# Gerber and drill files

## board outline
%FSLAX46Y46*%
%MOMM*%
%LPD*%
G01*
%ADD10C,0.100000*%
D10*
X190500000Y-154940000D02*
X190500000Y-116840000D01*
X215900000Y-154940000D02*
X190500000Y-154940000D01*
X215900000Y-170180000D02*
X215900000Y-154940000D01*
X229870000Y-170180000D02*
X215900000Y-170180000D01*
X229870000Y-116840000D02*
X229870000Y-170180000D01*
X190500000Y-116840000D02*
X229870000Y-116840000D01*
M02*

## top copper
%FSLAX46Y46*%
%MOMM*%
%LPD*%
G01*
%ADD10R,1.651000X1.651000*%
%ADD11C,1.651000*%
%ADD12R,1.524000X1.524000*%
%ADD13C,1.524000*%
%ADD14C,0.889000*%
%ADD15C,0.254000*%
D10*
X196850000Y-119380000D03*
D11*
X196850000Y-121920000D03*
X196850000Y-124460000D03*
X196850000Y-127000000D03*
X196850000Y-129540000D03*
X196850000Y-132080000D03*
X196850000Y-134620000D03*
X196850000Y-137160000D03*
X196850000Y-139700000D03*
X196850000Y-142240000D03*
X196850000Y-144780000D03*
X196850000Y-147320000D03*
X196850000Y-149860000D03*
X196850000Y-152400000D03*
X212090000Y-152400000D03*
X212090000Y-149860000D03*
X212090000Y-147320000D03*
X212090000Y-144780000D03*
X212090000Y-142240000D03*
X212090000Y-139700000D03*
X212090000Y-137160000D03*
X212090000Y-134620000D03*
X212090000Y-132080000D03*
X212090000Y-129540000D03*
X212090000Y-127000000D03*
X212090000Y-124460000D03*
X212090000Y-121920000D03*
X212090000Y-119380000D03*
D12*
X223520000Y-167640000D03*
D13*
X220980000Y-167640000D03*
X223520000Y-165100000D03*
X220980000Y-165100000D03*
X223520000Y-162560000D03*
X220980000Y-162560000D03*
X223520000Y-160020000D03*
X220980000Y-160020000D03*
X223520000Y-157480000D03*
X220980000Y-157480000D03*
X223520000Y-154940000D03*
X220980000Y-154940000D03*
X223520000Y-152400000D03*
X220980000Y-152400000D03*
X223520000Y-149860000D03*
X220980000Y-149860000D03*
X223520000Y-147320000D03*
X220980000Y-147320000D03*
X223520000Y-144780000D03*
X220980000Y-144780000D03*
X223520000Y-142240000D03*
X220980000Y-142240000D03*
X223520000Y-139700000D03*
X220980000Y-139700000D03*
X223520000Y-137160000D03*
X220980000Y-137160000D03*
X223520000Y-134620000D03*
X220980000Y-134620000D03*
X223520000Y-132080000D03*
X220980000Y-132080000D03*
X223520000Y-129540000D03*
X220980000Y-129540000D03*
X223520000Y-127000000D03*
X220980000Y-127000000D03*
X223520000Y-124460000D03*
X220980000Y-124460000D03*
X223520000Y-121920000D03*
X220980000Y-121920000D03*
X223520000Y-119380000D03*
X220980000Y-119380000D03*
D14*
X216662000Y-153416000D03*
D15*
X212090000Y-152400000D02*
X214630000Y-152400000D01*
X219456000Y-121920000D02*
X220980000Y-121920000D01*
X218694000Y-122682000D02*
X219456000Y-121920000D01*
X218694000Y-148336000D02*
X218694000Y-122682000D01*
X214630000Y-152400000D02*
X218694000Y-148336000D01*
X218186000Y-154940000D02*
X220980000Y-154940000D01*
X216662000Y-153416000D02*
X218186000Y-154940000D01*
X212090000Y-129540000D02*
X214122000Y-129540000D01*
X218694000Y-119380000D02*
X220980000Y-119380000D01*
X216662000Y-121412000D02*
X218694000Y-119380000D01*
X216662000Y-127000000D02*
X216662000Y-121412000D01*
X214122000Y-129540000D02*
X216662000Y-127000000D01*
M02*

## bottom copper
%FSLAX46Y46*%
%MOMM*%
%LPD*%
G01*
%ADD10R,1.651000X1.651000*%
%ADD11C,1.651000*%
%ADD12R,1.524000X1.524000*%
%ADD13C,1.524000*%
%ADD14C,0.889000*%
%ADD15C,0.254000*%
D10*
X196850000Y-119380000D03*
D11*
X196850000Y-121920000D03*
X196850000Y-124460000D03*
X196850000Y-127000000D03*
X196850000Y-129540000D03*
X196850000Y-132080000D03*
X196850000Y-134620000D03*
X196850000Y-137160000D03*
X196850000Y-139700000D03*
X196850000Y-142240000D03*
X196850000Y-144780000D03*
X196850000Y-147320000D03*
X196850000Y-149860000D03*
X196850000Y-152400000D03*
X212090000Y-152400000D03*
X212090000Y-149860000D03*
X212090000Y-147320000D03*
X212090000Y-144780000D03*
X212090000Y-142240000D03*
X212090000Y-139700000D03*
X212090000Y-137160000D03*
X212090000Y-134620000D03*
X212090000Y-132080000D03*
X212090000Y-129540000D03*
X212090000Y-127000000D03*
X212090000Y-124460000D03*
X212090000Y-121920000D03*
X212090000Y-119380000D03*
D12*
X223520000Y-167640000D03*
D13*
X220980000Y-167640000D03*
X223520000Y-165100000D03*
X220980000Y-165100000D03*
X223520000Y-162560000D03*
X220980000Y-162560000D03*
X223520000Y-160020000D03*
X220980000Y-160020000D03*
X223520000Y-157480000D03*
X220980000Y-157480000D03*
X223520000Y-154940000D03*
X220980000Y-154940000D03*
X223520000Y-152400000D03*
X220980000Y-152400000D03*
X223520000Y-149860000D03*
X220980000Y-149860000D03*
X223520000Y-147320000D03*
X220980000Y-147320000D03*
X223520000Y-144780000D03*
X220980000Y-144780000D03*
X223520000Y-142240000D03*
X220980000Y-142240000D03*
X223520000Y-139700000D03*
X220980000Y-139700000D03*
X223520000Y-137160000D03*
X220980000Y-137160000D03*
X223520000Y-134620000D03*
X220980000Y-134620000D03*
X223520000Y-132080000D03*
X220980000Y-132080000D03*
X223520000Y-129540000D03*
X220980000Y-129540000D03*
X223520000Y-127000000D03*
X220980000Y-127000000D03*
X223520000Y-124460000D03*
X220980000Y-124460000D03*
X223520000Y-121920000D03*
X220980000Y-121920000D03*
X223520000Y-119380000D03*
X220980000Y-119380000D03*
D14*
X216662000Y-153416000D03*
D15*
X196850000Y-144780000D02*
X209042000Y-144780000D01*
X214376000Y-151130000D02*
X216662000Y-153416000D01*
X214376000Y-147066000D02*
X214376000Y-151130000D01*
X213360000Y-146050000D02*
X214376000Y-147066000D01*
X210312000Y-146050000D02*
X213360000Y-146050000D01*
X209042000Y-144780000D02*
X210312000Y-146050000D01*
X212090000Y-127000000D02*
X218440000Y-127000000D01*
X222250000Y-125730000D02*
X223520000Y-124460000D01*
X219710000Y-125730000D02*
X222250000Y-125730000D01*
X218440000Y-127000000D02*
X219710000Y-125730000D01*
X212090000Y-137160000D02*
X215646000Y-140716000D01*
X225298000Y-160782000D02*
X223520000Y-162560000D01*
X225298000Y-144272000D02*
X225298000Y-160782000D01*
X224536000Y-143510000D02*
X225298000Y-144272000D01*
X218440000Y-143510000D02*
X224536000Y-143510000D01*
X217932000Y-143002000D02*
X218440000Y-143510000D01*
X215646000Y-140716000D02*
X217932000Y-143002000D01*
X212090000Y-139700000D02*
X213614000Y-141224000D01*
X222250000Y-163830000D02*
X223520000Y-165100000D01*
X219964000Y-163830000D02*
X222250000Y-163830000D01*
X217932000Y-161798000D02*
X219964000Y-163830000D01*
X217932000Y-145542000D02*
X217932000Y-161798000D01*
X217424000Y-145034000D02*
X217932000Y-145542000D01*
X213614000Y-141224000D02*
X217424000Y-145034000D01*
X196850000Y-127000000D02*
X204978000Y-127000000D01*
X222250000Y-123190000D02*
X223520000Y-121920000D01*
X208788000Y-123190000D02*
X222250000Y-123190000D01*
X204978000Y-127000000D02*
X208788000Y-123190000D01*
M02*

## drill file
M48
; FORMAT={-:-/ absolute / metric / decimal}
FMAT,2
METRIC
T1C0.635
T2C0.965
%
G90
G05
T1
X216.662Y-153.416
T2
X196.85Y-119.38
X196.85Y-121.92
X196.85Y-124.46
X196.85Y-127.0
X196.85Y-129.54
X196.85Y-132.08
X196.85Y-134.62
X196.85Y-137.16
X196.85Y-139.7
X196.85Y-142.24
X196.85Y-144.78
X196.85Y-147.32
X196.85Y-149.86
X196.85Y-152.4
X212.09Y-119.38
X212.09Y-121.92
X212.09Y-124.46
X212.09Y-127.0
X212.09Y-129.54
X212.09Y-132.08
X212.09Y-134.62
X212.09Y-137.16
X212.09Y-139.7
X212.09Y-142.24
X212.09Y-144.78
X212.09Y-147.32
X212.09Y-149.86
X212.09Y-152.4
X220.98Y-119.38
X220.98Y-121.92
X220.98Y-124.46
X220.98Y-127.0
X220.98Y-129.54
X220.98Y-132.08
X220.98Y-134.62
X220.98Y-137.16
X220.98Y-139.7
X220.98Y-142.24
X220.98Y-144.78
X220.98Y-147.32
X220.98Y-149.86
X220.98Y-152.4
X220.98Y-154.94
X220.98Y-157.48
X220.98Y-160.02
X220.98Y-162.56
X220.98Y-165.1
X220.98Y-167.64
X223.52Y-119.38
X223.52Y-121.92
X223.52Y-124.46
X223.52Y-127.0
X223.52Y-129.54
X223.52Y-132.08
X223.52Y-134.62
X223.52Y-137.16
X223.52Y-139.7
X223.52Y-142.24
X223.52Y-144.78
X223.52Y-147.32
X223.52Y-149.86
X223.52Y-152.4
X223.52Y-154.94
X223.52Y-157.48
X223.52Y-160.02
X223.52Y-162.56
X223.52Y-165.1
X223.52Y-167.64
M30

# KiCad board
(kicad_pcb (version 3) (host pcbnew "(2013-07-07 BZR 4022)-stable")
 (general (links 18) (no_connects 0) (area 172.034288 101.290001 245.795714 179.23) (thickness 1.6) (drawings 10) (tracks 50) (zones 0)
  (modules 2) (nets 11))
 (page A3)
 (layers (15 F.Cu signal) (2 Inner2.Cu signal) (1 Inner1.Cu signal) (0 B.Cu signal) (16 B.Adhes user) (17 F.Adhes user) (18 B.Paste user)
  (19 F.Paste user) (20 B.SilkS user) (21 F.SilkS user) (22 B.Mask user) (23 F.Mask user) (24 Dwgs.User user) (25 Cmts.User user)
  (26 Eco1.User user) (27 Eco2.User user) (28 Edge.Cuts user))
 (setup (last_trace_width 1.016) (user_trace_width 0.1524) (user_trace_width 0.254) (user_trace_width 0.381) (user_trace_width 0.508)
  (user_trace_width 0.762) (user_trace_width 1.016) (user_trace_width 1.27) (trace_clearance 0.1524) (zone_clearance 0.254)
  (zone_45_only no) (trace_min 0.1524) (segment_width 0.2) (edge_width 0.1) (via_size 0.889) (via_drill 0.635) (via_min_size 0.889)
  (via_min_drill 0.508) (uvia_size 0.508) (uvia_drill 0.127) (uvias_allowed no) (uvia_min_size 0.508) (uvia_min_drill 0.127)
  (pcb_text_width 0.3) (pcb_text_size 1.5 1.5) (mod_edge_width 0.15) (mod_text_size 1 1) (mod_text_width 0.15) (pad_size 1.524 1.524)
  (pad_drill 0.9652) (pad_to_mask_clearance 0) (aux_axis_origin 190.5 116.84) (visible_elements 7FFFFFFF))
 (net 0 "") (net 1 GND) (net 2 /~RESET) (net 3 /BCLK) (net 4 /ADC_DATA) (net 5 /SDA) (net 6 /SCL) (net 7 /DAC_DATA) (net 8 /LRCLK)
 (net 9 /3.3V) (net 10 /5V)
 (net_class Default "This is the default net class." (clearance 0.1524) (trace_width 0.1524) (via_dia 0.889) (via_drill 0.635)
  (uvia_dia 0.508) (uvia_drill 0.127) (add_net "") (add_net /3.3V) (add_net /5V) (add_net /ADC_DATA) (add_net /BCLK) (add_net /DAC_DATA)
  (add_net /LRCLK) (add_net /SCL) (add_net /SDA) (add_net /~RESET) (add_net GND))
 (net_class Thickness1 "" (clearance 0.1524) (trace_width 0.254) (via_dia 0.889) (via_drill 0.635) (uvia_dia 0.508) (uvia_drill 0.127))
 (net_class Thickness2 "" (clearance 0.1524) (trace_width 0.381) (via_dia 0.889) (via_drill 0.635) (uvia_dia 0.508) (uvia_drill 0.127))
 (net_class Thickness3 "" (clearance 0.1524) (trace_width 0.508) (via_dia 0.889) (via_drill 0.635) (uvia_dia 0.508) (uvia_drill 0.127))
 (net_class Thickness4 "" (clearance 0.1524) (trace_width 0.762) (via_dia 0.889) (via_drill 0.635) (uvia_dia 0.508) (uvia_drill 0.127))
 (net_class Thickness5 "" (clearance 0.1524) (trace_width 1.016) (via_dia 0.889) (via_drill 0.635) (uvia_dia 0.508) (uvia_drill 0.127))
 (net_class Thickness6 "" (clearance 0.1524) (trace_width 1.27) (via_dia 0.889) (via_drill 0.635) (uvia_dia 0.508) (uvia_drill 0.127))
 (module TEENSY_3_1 (layer F.Cu) (at 204.47 135.89)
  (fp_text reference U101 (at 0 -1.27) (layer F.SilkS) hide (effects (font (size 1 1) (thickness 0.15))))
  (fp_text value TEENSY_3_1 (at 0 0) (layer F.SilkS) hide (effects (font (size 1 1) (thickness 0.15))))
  (pad 1 thru_hole rect (at -7.62 -16.51) (size 1.651 1.651) (drill 0.9652) (layers *.Cu *.Mask F.SilkS) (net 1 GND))
  (pad 2 thru_hole circle (at -7.62 -13.97) (size 1.651 1.651) (drill 0.9652) (layers *.Cu *.Mask F.SilkS))
  (pad 3 thru_hole circle (at -7.62 -11.43) (size 1.651 1.651) (drill 0.9652) (layers *.Cu *.Mask F.SilkS))
  (pad 4 thru_hole circle (at -7.62 -8.89) (size 1.651 1.651) (drill 0.9652) (layers *.Cu *.Mask F.SilkS) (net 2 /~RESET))
  (pad 5 thru_hole circle (at -7.62 -6.35) (size 1.651 1.651) (drill 0.9652) (layers *.Cu *.Mask F.SilkS))
  (pad 6 thru_hole circle (at -7.62 -3.81) (size 1.651 1.651) (drill 0.9652) (layers *.Cu *.Mask F.SilkS))
  (pad 7 thru_hole circle (at -7.62 -1.27) (size 1.651 1.651) (drill 0.9652) (layers *.Cu *.Mask F.SilkS))
  (pad 8 thru_hole circle (at -7.62 1.27) (size 1.651 1.651) (drill 0.9652) (layers *.Cu *.Mask F.SilkS))
  (pad 9 thru_hole circle (at -7.62 3.81) (size 1.651 1.651) (drill 0.9652) (layers *.Cu *.Mask F.SilkS))
  (pad 10 thru_hole circle (at -7.62 6.35) (size 1.651 1.651) (drill 0.9652) (layers *.Cu *.Mask F.SilkS))
  (pad 11 thru_hole circle (at -7.62 8.89) (size 1.651 1.651) (drill 0.9652) (layers *.Cu *.Mask F.SilkS) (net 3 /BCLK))
  (pad 12 thru_hole circle (at -7.62 11.43) (size 1.651 1.651) (drill 0.9652) (layers *.Cu *.Mask F.SilkS))
  (pad 13 thru_hole circle (at -7.62 13.97) (size 1.651 1.651) (drill 0.9652) (layers *.Cu *.Mask F.SilkS))
  (pad 14 thru_hole circle (at -7.62 16.51) (size 1.651 1.651) (drill 0.9652) (layers *.Cu *.Mask F.SilkS))
  (pad 20 thru_hole circle (at 7.62 16.51) (size 1.651 1.651) (drill 0.9652) (layers *.Cu *.Mask F.SilkS) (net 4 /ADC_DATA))
  (pad 21 thru_hole circle (at 7.62 13.97) (size 1.651 1.651) (drill 0.9652) (layers *.Cu *.Mask F.SilkS))
  (pad 22 thru_hole circle (at 7.62 11.43) (size 1.651 1.651) (drill 0.9652) (layers *.Cu *.Mask F.SilkS))
  (pad 23 thru_hole circle (at 7.62 8.89) (size 1.651 1.651) (drill 0.9652) (layers *.Cu *.Mask F.SilkS))
  (pad 24 thru_hole circle (at 7.62 6.35) (size 1.651 1.651) (drill 0.9652) (layers *.Cu *.Mask F.SilkS))
  (pad 25 thru_hole circle (at 7.62 3.81) (size 1.651 1.651) (drill 0.9652) (layers *.Cu *.Mask F.SilkS) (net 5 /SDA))
  (pad 26 thru_hole circle (at 7.62 1.27) (size 1.651 1.651) (drill 0.9652) (layers *.Cu *.Mask F.SilkS) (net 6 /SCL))
  (pad 27 thru_hole circle (at 7.62 -1.27) (size 1.651 1.651) (drill 0.9652) (layers *.Cu *.Mask F.SilkS))
  (pad 28 thru_hole circle (at 7.62 -3.81) (size 1.651 1.651) (drill 0.9652) (layers *.Cu *.Mask F.SilkS))
  (pad 29 thru_hole circle (at 7.62 -6.35) (size 1.651 1.651) (drill 0.9652) (layers *.Cu *.Mask F.SilkS) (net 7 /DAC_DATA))
  (pad 30 thru_hole circle (at 7.62 -8.89) (size 1.651 1.651) (drill 0.9652) (layers *.Cu *.Mask F.SilkS) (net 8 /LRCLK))
  (pad 31 thru_hole circle (at 7.62 -11.43) (size 1.651 1.651) (drill 0.9652) (layers *.Cu *.Mask F.SilkS) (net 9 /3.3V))
  (pad 32 thru_hole circle (at 7.62 -13.97) (size 1.651 1.651) (drill 0.9652) (layers *.Cu *.Mask F.SilkS))
  (pad 33 thru_hole circle (at 7.62 -16.51) (size 1.651 1.651) (drill 0.9652) (layers *.Cu *.Mask F.SilkS) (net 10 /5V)))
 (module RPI (layer F.Cu) (at 222.25 143.51 180)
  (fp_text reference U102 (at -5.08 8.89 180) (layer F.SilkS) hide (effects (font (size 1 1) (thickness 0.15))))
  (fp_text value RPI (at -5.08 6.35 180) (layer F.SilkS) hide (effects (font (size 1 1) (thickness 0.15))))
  (pad 1 thru_hole rect (at -1.27 -24.13 180) (size 1.524 1.524) (drill 0.9652) (layers *.Cu *.Mask F.SilkS) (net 9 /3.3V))
  (pad 2 thru_hole circle (at 1.27 -24.13 180) (size 1.524 1.524) (drill 0.9652) (layers *.Cu *.Mask F.SilkS) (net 10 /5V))
  (pad 3 thru_hole circle (at -1.27 -21.59 180) (size 1.524 1.524) (drill 0.9652) (layers *.Cu *.Mask F.SilkS) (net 5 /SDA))
  (pad 4 thru_hole circle (at 1.27 -21.59 180) (size 1.524 1.524) (drill 0.9652) (layers *.Cu *.Mask F.SilkS) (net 10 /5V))
  (pad 5 thru_hole circle (at -1.27 -19.05 180) (size 1.524 1.524) (drill 0.9652) (layers *.Cu *.Mask F.SilkS) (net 6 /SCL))
  (pad 6 thru_hole circle (at 1.27 -19.05 180) (size 1.524 1.524) (drill 0.9652) (layers *.Cu *.Mask F.SilkS) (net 1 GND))
  (pad 7 thru_hole circle (at -1.27 -16.51 180) (size 1.524 1.524) (drill 0.9652) (layers *.Cu *.Mask F.SilkS))
  (pad 8 thru_hole circle (at 1.27 -16.51 180) (size 1.524 1.524) (drill 0.9652) (layers *.Cu *.Mask F.SilkS))
  (pad 9 thru_hole circle (at -1.27 -13.97 180) (size 1.524 1.524) (drill 0.9652) (layers *.Cu *.Mask F.SilkS) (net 1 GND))
  (pad 10 thru_hole circle (at 1.27 -13.97 180) (size 1.524 1.524) (drill 0.9652) (layers *.Cu *.Mask F.SilkS))
  (pad 11 thru_hole circle (at -1.27 -11.43 180) (size 1.524 1.524) (drill 0.9652) (layers *.Cu *.Mask F.SilkS))
  (pad 12 thru_hole circle (at 1.27 -11.43 180) (size 1.524 1.524) (drill 0.9652) (layers *.Cu *.Mask F.SilkS) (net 3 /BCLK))
  (pad 13 thru_hole circle (at -1.27 -8.89 180) (size 1.524 1.524) (drill 0.9652) (layers *.Cu *.Mask F.SilkS))
  (pad 14 thru_hole circle (at 1.27 -8.89 180) (size 1.524 1.524) (drill 0.9652) (layers *.Cu *.Mask F.SilkS) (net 1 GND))
  (pad 15 thru_hole circle (at -1.27 -6.35 180) (size 1.524 1.524) (drill 0.9652) (layers *.Cu *.Mask F.SilkS))
  (pad 16 thru_hole circle (at 1.27 -6.35 180) (size 1.524 1.524) (drill 0.9652) (layers *.Cu *.Mask F.SilkS))
  (pad 17 thru_hole circle (at -1.27 -3.81 180) (size 1.524 1.524) (drill 0.9652) (layers *.Cu *.Mask F.SilkS))
  (pad 18 thru_hole circle (at 1.27 -3.81 180) (size 1.524 1.524) (drill 0.9652) (layers *.Cu *.Mask F.SilkS))
  (pad 19 thru_hole circle (at -1.27 -1.27 180) (size 1.524 1.524) (drill 0.9652) (layers *.Cu *.Mask F.SilkS))
  (pad 20 thru_hole circle (at 1.27 -1.27 180) (size 1.524 1.524) (drill 0.9652) (layers *.Cu *.Mask F.SilkS) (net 1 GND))
  (pad 21 thru_hole circle (at -1.27 1.27 180) (size 1.524 1.524) (drill 0.9652) (layers *.Cu *.Mask F.SilkS))
  (pad 22 thru_hole circle (at 1.27 1.27 180) (size 1.524 1.524) (drill 0.9652) (layers *.Cu *.Mask F.SilkS))
  (pad 23 thru_hole circle (at -1.27 3.81 180) (size 1.524 1.524) (drill 0.9652) (layers *.Cu *.Mask F.SilkS))
  (pad 24 thru_hole circle (at 1.27 3.81 180) (size 1.524 1.524) (drill 0.9652) (layers *.Cu *.Mask F.SilkS))
  (pad 25 thru_hole circle (at -1.27 6.35 180) (size 1.524 1.524) (drill 0.9652) (layers *.Cu *.Mask F.SilkS) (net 1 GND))
  (pad 26 thru_hole circle (at 1.27 6.35 180) (size 1.524 1.524) (drill 0.9652) (layers *.Cu *.Mask F.SilkS))
  (pad 27 thru_hole circle (at -1.27 8.89 180) (size 1.524 1.524) (drill 0.9652) (layers *.Cu *.Mask F.SilkS))
  (pad 28 thru_hole circle (at 1.27 8.89 180) (size 1.524 1.524) (drill 0.9652) (layers *.Cu *.Mask F.SilkS))
  (pad 29 thru_hole circle (at -1.27 11.43 180) (size 1.524 1.524) (drill 0.9652) (layers *.Cu *.Mask F.SilkS))
  (pad 30 thru_hole circle (at 1.27 11.43 180) (size 1.524 1.524) (drill 0.9652) (layers *.Cu *.Mask F.SilkS) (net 1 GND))
  (pad 31 thru_hole circle (at -1.27 13.97 180) (size 1.524 1.524) (drill 0.9652) (layers *.Cu *.Mask F.SilkS))
  (pad 32 thru_hole circle (at 1.27 13.97 180) (size 1.524 1.524) (drill 0.9652) (layers *.Cu *.Mask F.SilkS))
  (pad 33 thru_hole circle (at -1.27 16.51 180) (size 1.524 1.524) (drill 0.9652) (layers *.Cu *.Mask F.SilkS))
  (pad 34 thru_hole circle (at 1.27 16.51 180) (size 1.524 1.524) (drill 0.9652) (layers *.Cu *.Mask F.SilkS) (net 1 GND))
  (pad 35 thru_hole circle (at -1.27 19.05 180) (size 1.524 1.524) (drill 0.9652) (layers *.Cu *.Mask F.SilkS) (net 8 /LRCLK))
  (pad 36 thru_hole circle (at 1.27 19.05 180) (size 1.524 1.524) (drill 0.9652) (layers *.Cu *.Mask F.SilkS))
  (pad 37 thru_hole circle (at -1.27 21.59 180) (size 1.524 1.524) (drill 0.9652) (layers *.Cu *.Mask F.SilkS) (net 2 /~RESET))
  (pad 38 thru_hole circle (at 1.27 21.59 180) (size 1.524 1.524) (drill 0.9652) (layers *.Cu *.Mask F.SilkS) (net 4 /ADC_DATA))
  (pad 39 thru_hole circle (at -1.27 24.13 180) (size 1.524 1.524) (drill 0.9652) (layers *.Cu *.Mask F.SilkS) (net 1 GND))
  (pad 40 thru_hole circle (at 1.27 24.13 180) (size 1.524 1.524) (drill 0.9652) (layers *.Cu *.Mask F.SilkS) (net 7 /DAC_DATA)))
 (gr_line (start 190.5 154.94) (end 190.5 116.84) (angle 90) (layer Edge.Cuts) (width 0.1))
 (gr_line (start 215.9 154.94) (end 190.5 154.94) (angle 90) (layer Edge.Cuts) (width 0.1))
 (gr_line (start 215.9 170.18) (end 215.9 154.94) (angle 90) (layer Edge.Cuts) (width 0.1))
 (gr_line (start 229.87 170.18) (end 215.9 170.18) (angle 90) (layer Edge.Cuts) (width 0.1))
 (gr_line (start 229.87 116.84) (end 229.87 170.18) (angle 90) (layer Edge.Cuts) (width 0.1))
 (gr_line (start 190.5 116.84) (end 229.87 116.84) (angle 90) (layer Edge.Cuts) (width 0.1))
 (segment (start 212.09 124.46) (end 215.392 124.46) (width 0.508) (layer Inner1.Cu) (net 9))
 (segment (start 225.044 167.64) (end 223.52 167.64) (width 0.508) (layer Inner1.Cu) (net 9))
 (segment (start 225.806 166.878) (end 225.044 167.64) (width 0.508) (layer Inner1.Cu) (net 9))
 (segment (start 225.806 131.826) (end 225.806 166.878) (width 0.508) (layer Inner1.Cu) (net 9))
 (segment (start 224.79 130.81) (end 225.806 131.826) (width 0.508) (layer Inner1.Cu) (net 9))
 (segment (start 219.202 130.81) (end 224.79 130.81) (width 0.508) (layer Inner1.Cu) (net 9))
 (segment (start 217.678 129.286) (end 219.202 130.81) (width 0.508) (layer Inner1.Cu) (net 9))
 (segment (start 217.678 126.746) (end 217.678 129.286) (width 0.508) (layer Inner1.Cu) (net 9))
 (segment (start 215.392 124.46) (end 217.678 126.746) (width 0.508) (layer Inner1.Cu) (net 9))
 (segment (start 212.09 152.4) (end 214.63 152.4) (width 0.254) (layer F.Cu) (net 4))
 (segment (start 219.456 121.92) (end 220.98 121.92) (width 0.254) (layer F.Cu) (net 4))
 (segment (start 218.694 122.682) (end 219.456 121.92) (width 0.254) (layer F.Cu) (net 4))
 (segment (start 218.694 148.336) (end 218.694 122.682) (width 0.254) (layer F.Cu) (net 4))
 (segment (start 214.63 152.4) (end 218.694 148.336) (width 0.254) (layer F.Cu) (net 4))
 (segment (start 196.85 144.78) (end 209.042 144.78) (width 0.254) (layer B.Cu) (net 3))
 (segment (start 218.186 154.94) (end 220.98 154.94) (width 0.254) (layer F.Cu) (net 3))
 (segment (start 216.662 153.416) (end 218.186 154.94) (width 0.254) (layer F.Cu) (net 3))
 (via (at 216.662 153.416) (size 0.889) (layers F.Cu B.Cu) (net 3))
 (segment (start 214.376 151.13) (end 216.662 153.416) (width 0.254) (layer B.Cu) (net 3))
 (segment (start 214.376 147.066) (end 214.376 151.13) (width 0.254) (layer B.Cu) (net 3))
 (segment (start 213.36 146.05) (end 214.376 147.066) (width 0.254) (layer B.Cu) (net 3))
 (segment (start 210.312 146.05) (end 213.36 146.05) (width 0.254) (layer B.Cu) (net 3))
 (segment (start 209.042 144.78) (end 210.312 146.05) (width 0.254) (layer B.Cu) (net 3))
 (segment (start 212.09 129.54) (end 214.122 129.54) (width 0.254) (layer F.Cu) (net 7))
 (segment (start 218.694 119.38) (end 220.98 119.38) (width 0.254) (layer F.Cu) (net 7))
 (segment (start 216.662 121.412) (end 218.694 119.38) (width 0.254) (layer F.Cu) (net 7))
 (segment (start 216.662 127) (end 216.662 121.412) (width 0.254) (layer F.Cu) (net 7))
 (segment (start 214.122 129.54) (end 216.662 127) (width 0.254) (layer F.Cu) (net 7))
 (segment (start 212.09 127) (end 218.44 127) (width 0.254) (layer B.Cu) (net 8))
 (segment (start 222.25 125.73) (end 223.52 124.46) (width 0.254) (layer B.Cu) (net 8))
 (segment (start 219.71 125.73) (end 222.25 125.73) (width 0.254) (layer B.Cu) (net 8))
 (segment (start 218.44 127) (end 219.71 125.73) (width 0.254) (layer B.Cu) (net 8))
 (segment (start 212.09 137.16) (end 215.646 140.716) (width 0.254) (layer B.Cu) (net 6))
 (segment (start 225.298 160.782) (end 223.52 162.56) (width 0.254) (layer B.Cu) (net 6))
 (segment (start 225.298 144.272) (end 225.298 160.782) (width 0.254) (layer B.Cu) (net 6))
 (segment (start 224.536 143.51) (end 225.298 144.272) (width 0.254) (layer B.Cu) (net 6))
 (segment (start 218.44 143.51) (end 224.536 143.51) (width 0.254) (layer B.Cu) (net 6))
 (segment (start 217.932 143.002) (end 218.44 143.51) (width 0.254) (layer B.Cu) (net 6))
 (segment (start 215.646 140.716) (end 217.932 143.002) (width 0.254) (layer B.Cu) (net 6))
 (segment (start 212.09 139.7) (end 213.614 141.224) (width 0.254) (layer B.Cu) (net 5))
 (segment (start 222.25 163.83) (end 223.52 165.1) (width 0.254) (layer B.Cu) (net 5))
 (segment (start 219.964 163.83) (end 222.25 163.83) (width 0.254) (layer B.Cu) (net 5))
 (segment (start 217.932 161.798) (end 219.964 163.83) (width 0.254) (layer B.Cu) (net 5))
 (segment (start 217.932 145.542) (end 217.932 161.798) (width 0.254) (layer B.Cu) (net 5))
 (segment (start 217.424 145.034) (end 217.932 145.542) (width 0.254) (layer B.Cu) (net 5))
 (segment (start 213.614 141.224) (end 217.424 145.034) (width 0.254) (layer B.Cu) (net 5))
 (segment (start 196.85 127) (end 204.978 127) (width 0.254) (layer B.Cu) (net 2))
 (segment (start 222.25 123.19) (end 223.52 121.92) (width 0.254) (layer B.Cu) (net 2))
 (segment (start 208.788 123.19) (end 222.25 123.19) (width 0.254) (layer B.Cu) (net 2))
 (segment (start 204.978 127) (end 208.788 123.19) (width 0.254) (layer B.Cu) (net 2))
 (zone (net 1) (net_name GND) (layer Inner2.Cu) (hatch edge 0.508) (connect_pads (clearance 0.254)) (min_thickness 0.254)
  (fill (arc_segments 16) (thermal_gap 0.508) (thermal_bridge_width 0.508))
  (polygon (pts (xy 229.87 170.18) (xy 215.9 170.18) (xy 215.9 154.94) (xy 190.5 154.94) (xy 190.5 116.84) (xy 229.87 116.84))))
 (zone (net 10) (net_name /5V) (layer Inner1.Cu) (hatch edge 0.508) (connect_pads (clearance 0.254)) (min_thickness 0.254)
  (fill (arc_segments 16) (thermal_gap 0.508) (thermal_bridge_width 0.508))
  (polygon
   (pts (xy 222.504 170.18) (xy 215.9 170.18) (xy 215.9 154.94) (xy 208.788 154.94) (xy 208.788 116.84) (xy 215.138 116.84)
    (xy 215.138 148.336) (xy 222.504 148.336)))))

